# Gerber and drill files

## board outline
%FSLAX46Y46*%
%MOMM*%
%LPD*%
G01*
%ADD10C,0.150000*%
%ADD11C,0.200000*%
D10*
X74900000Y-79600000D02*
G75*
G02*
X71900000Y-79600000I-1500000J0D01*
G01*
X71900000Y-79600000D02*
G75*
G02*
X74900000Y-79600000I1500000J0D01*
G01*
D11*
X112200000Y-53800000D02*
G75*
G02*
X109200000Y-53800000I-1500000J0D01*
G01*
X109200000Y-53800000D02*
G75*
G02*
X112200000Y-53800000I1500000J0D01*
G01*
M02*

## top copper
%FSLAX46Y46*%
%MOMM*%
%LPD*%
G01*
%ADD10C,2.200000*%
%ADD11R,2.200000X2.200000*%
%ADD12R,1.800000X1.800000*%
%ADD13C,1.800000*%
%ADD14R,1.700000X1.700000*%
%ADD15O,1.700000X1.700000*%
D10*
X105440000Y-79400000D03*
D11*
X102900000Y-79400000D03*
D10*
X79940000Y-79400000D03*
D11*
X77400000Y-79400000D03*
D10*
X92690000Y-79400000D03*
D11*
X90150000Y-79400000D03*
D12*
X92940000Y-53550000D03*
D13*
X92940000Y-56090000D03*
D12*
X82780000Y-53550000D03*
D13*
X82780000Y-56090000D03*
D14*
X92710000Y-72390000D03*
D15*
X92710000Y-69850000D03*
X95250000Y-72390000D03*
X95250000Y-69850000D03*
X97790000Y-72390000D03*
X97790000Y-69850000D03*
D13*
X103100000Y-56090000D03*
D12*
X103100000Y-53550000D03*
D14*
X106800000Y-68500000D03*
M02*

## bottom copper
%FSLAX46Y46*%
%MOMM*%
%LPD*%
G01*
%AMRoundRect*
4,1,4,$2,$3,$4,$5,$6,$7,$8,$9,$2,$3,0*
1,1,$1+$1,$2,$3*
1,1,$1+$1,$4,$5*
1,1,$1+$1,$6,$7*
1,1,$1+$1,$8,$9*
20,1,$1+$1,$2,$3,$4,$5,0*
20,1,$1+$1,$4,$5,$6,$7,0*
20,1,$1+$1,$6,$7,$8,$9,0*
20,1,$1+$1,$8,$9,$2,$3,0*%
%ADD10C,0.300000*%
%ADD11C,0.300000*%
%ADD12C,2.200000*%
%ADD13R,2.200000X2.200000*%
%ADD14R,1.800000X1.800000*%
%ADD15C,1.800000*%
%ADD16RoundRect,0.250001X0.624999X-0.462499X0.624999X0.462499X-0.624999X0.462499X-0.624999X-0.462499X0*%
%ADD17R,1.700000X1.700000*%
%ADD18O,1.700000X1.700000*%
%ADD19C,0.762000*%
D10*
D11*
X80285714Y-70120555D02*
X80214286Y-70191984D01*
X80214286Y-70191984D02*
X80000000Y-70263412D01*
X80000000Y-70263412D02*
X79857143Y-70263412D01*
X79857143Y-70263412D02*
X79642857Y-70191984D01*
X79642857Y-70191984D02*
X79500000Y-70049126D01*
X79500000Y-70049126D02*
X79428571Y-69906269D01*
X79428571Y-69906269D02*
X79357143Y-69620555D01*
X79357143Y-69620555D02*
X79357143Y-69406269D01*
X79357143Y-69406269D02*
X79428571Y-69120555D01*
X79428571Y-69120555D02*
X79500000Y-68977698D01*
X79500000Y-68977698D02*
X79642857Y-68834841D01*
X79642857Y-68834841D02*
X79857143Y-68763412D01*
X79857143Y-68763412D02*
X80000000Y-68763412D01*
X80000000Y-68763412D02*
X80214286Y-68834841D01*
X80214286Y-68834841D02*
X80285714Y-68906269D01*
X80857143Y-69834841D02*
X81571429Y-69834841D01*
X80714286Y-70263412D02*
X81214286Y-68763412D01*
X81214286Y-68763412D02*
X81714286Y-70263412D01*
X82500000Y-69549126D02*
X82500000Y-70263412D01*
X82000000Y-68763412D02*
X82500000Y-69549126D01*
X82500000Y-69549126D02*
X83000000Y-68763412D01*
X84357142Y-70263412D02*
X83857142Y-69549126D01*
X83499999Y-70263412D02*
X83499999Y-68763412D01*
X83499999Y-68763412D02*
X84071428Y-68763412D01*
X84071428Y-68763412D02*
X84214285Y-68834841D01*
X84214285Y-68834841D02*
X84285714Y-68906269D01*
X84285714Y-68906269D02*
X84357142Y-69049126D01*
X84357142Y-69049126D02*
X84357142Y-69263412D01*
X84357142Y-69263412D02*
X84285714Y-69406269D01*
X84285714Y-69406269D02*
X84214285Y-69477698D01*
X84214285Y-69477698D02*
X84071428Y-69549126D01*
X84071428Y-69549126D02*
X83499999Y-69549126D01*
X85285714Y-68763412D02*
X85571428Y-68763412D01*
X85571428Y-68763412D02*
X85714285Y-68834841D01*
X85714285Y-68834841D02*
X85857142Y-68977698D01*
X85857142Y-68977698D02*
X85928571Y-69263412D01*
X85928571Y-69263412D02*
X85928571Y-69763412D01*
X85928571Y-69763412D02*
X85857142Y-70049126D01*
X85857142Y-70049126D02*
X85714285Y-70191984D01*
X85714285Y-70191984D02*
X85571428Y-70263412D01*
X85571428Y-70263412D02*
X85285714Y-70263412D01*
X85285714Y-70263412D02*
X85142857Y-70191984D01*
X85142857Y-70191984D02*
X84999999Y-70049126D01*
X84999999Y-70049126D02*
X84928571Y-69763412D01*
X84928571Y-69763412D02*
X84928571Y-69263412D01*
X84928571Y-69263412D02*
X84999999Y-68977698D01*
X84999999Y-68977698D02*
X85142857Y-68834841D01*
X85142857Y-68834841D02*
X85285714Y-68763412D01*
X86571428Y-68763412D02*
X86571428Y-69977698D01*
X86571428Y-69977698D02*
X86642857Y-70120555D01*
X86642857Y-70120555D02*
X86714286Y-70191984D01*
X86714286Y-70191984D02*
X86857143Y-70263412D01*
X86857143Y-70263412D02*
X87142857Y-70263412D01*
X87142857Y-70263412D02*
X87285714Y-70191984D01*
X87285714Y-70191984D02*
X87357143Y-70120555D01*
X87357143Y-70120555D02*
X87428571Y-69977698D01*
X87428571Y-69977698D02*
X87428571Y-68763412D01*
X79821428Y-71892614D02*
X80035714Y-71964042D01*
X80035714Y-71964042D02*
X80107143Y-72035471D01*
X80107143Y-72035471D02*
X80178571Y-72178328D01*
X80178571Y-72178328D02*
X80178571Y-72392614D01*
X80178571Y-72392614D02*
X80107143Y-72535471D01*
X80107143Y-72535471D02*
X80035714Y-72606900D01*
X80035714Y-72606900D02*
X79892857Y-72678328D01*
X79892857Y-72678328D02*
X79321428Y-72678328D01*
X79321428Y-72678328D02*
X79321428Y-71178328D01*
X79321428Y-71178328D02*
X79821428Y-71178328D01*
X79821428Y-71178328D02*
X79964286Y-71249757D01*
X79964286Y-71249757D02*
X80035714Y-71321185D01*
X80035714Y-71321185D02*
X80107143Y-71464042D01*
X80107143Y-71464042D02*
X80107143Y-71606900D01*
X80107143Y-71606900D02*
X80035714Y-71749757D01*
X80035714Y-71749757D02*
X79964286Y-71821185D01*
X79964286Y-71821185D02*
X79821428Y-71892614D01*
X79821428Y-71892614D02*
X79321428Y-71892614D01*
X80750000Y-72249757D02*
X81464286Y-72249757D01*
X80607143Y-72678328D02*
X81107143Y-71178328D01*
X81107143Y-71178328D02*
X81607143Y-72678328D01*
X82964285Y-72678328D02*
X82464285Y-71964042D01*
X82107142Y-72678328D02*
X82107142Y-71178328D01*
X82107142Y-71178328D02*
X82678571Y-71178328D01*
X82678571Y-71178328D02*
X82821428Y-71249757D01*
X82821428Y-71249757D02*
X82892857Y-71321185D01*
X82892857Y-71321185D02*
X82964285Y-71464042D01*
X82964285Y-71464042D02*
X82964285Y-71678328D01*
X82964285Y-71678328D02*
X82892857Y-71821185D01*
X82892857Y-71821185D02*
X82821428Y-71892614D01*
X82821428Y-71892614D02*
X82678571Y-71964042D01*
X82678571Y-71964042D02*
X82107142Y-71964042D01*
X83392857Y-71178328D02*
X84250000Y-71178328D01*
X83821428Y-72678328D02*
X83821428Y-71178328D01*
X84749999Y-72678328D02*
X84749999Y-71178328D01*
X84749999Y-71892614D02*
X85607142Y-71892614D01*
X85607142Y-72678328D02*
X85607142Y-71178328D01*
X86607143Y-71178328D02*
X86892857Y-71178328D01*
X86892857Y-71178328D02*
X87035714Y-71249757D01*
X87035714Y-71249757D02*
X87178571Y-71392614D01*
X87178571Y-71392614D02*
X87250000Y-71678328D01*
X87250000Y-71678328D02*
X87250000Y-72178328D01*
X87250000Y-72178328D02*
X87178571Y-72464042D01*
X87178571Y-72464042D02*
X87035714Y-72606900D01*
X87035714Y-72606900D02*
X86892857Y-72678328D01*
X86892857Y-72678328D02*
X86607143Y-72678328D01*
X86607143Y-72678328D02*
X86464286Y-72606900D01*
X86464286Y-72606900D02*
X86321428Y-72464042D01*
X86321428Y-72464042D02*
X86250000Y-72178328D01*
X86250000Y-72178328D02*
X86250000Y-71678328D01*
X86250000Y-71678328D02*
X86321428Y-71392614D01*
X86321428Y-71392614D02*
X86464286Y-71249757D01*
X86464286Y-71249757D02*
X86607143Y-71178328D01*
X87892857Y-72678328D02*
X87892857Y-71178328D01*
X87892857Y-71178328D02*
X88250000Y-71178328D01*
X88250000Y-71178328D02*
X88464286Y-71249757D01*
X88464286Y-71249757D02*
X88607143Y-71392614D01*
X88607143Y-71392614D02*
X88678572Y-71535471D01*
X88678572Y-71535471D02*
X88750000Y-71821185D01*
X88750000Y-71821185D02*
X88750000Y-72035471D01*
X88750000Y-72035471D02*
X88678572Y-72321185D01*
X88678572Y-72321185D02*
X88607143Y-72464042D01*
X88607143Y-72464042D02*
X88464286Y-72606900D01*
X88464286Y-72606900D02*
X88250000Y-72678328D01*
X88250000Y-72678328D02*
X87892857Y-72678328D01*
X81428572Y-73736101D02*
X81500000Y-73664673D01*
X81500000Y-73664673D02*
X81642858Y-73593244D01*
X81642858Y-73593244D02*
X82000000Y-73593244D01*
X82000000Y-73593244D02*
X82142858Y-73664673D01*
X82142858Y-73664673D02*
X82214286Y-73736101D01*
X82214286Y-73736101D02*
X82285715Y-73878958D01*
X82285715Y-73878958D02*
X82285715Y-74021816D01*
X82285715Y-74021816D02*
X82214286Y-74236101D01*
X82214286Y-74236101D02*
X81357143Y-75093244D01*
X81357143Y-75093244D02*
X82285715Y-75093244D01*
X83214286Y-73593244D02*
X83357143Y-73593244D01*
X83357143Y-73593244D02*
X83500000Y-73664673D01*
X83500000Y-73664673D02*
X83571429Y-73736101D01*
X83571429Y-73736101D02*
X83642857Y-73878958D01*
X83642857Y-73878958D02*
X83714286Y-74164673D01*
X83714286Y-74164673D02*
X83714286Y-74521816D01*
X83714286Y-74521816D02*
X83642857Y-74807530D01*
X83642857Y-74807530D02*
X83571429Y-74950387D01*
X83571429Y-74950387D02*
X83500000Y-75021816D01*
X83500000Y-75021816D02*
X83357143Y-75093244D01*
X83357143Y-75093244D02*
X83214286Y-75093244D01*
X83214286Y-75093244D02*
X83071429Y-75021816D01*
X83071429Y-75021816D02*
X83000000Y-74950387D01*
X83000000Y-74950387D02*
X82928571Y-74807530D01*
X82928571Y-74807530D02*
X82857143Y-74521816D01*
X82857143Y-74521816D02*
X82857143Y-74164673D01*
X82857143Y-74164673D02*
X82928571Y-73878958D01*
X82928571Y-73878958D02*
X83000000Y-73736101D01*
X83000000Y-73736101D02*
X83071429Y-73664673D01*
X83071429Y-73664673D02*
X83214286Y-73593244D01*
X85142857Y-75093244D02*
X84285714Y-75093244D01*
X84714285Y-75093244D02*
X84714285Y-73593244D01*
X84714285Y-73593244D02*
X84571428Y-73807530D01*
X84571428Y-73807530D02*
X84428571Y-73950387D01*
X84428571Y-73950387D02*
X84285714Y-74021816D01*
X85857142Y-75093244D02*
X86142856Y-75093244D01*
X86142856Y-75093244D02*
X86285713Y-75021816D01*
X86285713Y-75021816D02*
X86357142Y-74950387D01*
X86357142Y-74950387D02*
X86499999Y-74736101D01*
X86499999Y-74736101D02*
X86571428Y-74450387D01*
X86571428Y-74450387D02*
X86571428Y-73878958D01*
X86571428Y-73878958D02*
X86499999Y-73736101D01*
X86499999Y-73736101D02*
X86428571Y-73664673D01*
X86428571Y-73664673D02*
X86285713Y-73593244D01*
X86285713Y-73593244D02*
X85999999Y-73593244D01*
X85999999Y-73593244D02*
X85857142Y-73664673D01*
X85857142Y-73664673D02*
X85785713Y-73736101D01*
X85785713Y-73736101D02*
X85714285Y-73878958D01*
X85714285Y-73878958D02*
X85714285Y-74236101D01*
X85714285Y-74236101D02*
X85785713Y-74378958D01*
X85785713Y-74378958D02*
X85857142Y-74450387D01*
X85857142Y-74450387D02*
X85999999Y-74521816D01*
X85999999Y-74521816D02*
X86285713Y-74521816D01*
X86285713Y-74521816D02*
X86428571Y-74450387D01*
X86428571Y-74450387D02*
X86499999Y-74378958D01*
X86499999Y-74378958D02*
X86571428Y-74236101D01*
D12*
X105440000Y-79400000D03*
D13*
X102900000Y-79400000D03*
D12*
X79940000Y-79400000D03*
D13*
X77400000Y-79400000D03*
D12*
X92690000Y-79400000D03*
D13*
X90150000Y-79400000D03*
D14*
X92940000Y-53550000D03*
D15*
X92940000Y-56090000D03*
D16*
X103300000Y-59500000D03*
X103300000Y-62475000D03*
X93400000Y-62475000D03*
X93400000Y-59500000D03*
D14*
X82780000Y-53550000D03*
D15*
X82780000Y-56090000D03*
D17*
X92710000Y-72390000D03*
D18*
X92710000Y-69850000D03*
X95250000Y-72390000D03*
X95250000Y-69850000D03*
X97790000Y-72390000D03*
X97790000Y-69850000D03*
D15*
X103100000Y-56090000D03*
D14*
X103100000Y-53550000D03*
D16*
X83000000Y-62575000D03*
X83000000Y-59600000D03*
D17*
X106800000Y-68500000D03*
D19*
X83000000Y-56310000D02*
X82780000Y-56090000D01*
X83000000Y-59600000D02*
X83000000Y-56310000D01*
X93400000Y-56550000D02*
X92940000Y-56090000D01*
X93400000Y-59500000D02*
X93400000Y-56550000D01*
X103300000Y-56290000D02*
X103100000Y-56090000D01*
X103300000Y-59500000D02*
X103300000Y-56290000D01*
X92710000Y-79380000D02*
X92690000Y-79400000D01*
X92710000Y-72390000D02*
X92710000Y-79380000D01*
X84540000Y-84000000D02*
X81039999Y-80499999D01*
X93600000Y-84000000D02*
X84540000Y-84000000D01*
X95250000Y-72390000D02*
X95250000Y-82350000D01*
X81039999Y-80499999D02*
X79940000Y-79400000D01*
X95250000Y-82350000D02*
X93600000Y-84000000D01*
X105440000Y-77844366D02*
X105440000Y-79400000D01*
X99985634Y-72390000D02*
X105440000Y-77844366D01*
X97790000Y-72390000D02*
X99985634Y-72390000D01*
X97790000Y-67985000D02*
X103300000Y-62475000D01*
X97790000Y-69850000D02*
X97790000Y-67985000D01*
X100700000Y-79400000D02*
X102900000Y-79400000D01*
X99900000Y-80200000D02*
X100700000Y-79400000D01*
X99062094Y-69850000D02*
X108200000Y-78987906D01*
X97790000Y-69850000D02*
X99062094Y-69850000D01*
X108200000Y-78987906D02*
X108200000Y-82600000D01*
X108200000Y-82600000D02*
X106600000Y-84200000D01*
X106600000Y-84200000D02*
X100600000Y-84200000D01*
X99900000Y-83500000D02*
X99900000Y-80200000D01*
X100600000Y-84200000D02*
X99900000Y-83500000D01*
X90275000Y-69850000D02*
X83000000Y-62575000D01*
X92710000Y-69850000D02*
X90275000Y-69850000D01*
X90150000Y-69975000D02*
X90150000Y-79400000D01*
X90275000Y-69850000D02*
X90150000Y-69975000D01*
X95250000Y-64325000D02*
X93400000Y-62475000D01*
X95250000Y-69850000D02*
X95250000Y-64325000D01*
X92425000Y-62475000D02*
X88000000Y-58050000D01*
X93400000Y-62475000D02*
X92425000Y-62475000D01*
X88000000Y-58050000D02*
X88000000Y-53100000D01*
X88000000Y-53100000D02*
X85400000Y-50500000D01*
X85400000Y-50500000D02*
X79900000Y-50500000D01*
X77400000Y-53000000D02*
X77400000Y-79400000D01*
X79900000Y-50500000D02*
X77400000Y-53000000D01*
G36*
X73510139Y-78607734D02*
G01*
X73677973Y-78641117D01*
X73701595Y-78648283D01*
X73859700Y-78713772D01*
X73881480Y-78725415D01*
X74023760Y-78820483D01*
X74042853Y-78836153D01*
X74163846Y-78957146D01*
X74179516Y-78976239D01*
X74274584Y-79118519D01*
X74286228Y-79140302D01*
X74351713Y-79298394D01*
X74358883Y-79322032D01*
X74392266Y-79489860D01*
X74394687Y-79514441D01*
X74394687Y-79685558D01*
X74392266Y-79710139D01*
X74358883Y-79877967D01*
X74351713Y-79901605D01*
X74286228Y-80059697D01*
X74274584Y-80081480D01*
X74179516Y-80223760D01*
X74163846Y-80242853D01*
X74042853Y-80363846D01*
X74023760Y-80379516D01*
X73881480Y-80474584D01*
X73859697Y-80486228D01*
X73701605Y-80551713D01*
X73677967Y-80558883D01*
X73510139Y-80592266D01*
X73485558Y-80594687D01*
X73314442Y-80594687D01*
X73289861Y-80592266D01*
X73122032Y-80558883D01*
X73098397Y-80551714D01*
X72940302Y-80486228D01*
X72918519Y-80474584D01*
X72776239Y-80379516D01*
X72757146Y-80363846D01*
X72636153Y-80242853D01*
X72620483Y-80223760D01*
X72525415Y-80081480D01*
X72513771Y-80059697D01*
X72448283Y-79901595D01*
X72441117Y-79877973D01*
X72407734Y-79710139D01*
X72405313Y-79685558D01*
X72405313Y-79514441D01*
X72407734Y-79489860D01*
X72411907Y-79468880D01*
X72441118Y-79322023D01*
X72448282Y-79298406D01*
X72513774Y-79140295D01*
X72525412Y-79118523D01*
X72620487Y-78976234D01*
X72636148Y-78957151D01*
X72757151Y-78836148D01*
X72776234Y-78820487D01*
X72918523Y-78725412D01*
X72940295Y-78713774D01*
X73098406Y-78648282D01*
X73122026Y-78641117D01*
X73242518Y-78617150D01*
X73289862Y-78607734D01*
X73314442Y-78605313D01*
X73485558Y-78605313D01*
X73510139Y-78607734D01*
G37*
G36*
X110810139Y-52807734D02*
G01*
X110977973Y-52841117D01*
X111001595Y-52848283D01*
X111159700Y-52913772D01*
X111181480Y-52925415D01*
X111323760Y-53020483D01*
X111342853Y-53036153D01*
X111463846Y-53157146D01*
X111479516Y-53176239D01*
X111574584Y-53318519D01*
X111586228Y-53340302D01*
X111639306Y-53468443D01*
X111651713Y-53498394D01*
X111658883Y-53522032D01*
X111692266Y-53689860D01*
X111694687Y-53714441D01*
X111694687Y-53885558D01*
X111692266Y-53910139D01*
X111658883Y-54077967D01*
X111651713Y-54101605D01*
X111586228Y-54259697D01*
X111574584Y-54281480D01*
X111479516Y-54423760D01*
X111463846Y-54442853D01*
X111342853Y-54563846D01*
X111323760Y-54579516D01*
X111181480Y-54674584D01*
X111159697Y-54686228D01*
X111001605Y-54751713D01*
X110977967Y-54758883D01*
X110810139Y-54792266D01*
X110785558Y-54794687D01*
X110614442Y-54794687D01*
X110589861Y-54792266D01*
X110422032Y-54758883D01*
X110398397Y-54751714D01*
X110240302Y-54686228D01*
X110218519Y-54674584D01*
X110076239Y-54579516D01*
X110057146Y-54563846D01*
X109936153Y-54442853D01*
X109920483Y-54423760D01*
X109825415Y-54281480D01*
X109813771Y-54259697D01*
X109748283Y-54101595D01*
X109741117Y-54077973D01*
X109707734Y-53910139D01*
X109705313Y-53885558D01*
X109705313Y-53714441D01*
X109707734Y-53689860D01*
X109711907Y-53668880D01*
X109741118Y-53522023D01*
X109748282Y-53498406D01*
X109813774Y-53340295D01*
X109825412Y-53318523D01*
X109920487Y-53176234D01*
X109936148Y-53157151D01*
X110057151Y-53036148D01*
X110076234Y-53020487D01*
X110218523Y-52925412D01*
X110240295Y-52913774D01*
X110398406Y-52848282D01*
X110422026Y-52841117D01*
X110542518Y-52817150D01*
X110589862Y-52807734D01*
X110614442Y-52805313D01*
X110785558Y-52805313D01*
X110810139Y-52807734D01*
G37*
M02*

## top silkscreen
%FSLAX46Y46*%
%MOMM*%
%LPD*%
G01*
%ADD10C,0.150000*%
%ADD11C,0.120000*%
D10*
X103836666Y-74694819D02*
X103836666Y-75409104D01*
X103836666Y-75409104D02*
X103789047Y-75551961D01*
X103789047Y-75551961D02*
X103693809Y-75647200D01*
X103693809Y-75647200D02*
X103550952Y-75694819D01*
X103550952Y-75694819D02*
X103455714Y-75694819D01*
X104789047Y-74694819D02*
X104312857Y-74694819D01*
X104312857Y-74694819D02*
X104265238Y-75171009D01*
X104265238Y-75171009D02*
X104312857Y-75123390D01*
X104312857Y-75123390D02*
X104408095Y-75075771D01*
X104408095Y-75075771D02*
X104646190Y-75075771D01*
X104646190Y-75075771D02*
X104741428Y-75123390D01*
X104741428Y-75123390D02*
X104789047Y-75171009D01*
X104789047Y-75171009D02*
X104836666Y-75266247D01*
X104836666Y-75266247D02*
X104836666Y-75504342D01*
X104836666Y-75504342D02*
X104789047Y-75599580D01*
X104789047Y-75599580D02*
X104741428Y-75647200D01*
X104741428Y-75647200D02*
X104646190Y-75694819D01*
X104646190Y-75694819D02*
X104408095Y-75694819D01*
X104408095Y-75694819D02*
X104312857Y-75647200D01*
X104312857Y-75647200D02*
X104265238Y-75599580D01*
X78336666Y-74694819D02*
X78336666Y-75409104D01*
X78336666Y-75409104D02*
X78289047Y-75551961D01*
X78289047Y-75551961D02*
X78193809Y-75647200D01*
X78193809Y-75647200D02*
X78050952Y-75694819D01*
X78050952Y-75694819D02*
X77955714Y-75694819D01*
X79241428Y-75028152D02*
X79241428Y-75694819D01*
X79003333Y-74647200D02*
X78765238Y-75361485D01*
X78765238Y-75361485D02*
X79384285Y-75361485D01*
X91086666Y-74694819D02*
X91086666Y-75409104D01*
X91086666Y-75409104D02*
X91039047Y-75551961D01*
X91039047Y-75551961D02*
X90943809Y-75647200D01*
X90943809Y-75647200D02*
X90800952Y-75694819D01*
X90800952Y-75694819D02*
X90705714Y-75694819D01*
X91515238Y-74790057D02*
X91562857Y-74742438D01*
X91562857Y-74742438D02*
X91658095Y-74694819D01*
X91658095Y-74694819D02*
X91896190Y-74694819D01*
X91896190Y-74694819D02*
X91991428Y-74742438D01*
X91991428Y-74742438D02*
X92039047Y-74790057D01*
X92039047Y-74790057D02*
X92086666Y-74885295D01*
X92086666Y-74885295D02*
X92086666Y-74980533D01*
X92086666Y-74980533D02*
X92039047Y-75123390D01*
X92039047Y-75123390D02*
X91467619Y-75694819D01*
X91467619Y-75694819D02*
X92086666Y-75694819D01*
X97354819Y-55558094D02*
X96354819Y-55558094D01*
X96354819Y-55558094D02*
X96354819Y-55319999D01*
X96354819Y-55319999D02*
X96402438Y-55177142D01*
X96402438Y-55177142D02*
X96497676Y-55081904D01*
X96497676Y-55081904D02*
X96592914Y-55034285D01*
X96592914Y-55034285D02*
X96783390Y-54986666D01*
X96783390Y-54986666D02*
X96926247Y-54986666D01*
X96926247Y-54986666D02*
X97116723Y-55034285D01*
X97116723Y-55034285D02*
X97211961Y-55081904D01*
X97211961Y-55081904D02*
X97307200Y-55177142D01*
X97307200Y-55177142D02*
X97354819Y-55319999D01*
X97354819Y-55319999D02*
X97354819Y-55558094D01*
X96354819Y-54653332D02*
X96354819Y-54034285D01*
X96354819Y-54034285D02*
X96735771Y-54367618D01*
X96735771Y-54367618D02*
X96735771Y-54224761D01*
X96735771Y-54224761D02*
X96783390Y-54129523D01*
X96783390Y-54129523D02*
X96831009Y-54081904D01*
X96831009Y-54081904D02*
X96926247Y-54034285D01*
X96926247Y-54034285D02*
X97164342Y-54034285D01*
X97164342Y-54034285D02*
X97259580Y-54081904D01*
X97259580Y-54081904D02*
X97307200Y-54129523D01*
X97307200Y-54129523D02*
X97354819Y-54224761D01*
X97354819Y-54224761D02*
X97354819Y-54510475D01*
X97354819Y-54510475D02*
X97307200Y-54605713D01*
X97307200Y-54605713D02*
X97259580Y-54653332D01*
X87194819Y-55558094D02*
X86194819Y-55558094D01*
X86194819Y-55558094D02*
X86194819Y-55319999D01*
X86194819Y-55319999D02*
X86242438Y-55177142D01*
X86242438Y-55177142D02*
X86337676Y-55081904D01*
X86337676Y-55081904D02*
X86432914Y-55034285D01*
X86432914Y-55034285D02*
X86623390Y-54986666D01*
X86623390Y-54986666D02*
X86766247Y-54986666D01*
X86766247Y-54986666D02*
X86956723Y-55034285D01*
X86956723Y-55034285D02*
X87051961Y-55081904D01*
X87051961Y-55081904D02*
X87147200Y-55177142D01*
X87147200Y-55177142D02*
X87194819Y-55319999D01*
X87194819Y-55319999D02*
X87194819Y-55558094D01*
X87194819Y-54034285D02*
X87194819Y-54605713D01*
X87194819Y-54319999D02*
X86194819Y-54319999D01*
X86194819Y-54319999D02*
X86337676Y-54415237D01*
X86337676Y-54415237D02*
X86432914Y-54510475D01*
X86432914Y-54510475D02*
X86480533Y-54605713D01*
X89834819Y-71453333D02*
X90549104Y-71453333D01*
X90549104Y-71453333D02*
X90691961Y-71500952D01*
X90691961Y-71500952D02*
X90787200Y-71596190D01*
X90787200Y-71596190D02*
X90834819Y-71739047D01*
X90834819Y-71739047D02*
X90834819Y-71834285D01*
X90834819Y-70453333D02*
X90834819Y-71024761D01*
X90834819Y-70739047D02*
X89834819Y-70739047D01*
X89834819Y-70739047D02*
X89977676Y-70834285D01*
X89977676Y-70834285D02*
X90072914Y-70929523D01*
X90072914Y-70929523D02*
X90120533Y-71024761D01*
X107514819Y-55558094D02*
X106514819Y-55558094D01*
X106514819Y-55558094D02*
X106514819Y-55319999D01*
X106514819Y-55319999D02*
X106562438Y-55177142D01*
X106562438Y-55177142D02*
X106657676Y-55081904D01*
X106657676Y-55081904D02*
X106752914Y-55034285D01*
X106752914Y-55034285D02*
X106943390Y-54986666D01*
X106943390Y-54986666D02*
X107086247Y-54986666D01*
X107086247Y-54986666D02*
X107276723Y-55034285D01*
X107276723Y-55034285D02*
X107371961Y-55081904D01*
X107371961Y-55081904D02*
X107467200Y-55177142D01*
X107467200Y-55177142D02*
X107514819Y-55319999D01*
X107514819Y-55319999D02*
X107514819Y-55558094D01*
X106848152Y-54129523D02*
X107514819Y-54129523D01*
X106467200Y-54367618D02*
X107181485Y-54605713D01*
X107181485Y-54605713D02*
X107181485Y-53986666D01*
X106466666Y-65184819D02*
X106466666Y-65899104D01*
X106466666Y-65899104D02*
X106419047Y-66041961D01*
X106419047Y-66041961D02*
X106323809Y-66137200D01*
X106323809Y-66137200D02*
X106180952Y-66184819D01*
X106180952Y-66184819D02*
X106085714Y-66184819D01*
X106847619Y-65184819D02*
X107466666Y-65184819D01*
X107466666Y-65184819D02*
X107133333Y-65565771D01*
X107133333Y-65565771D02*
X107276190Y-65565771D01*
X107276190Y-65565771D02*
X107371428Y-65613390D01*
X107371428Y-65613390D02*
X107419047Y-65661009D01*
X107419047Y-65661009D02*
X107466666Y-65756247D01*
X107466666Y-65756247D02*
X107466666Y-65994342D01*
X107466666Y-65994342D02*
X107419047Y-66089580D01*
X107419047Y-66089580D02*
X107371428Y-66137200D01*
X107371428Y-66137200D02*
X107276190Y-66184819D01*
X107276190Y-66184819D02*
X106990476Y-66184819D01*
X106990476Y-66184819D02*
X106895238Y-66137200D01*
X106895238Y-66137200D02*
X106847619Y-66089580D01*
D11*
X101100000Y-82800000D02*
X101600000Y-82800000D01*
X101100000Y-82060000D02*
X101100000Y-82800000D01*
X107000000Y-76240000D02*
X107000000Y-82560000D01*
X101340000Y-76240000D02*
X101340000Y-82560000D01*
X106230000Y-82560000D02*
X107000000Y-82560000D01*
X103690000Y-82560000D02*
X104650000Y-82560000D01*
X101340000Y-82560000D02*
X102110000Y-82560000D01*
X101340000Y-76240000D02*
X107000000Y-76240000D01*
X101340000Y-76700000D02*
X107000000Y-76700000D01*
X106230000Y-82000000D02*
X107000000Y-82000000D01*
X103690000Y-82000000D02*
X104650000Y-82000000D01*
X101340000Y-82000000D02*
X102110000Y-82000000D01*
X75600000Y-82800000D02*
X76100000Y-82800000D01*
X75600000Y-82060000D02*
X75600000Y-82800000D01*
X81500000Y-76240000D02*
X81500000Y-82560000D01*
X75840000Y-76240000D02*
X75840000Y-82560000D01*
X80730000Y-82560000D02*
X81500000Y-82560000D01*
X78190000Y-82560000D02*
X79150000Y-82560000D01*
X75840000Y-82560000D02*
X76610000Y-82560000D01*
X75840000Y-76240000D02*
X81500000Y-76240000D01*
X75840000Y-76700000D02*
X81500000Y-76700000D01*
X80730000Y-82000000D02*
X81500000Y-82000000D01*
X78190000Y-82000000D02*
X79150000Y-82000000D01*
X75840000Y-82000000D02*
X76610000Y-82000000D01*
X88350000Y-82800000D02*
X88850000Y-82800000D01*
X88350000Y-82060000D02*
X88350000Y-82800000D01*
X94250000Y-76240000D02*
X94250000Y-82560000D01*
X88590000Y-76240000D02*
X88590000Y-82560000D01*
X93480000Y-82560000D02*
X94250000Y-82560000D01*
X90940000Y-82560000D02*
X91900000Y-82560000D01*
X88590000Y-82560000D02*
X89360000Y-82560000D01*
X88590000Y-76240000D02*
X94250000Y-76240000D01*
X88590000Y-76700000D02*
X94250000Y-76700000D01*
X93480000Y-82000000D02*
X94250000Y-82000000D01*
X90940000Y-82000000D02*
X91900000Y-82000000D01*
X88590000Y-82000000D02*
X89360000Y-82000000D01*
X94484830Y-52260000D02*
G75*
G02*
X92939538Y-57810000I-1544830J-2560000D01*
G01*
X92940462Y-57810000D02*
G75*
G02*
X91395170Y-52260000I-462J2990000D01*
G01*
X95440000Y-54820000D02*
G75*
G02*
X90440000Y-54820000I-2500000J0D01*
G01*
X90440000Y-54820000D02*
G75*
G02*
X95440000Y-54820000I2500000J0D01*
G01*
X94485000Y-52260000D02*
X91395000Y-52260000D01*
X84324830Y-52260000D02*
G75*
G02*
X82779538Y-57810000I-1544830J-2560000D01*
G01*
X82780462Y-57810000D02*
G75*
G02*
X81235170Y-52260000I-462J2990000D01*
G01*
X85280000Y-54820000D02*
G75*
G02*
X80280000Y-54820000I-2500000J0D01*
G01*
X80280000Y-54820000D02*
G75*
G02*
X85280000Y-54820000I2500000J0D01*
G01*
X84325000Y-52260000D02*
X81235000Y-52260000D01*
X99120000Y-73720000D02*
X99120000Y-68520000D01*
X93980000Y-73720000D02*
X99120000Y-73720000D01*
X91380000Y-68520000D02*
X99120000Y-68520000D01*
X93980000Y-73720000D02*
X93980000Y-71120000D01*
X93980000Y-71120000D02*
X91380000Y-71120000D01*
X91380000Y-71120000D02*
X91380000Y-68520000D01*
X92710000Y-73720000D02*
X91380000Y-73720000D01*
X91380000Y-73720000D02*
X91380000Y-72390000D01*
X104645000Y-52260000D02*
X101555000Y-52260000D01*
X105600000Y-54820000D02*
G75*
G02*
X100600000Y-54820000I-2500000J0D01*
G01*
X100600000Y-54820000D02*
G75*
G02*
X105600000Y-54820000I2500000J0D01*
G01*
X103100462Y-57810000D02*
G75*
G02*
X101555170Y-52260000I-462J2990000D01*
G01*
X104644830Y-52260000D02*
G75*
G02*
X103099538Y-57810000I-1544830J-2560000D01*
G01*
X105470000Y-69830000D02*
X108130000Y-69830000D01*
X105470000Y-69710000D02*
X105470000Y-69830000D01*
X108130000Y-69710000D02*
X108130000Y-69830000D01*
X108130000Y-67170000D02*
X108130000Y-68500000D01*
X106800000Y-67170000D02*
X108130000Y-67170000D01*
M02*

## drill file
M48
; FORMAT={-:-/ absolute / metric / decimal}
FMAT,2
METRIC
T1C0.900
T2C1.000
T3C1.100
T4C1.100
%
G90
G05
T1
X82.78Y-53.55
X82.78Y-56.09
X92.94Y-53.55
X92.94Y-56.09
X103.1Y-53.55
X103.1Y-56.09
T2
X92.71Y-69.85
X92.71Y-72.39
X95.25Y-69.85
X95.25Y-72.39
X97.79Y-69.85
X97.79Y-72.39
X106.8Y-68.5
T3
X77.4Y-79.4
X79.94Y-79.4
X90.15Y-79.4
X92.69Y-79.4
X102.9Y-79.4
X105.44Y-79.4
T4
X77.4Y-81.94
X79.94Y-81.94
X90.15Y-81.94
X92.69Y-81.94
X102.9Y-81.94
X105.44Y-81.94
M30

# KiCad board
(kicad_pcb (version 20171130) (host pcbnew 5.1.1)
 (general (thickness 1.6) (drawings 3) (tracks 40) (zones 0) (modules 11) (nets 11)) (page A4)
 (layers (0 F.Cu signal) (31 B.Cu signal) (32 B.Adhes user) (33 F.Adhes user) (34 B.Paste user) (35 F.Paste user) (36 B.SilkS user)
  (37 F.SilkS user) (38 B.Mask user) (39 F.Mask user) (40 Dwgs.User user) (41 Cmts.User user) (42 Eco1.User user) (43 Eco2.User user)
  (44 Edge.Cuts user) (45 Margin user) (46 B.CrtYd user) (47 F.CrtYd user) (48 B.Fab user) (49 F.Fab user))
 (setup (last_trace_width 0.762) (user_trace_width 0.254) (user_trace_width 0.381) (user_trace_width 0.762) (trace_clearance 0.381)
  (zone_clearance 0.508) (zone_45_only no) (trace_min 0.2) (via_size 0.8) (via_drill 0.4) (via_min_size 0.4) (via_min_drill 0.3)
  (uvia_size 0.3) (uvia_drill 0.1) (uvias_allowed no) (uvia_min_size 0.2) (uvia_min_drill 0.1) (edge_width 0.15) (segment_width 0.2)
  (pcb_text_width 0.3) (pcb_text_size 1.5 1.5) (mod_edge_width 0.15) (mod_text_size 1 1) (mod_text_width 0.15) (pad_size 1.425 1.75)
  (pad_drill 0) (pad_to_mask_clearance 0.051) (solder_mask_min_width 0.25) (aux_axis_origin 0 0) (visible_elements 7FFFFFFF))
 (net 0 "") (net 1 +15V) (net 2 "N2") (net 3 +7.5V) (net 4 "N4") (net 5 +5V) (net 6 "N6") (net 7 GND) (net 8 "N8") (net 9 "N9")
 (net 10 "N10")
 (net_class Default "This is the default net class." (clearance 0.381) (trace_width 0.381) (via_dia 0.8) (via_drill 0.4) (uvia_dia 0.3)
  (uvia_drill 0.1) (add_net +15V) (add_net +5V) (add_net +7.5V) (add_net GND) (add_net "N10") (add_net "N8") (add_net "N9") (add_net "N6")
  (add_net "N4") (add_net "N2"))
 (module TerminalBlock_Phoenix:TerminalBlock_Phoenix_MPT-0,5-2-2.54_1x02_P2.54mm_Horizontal (layer F.Cu) (at 102.9 79.4)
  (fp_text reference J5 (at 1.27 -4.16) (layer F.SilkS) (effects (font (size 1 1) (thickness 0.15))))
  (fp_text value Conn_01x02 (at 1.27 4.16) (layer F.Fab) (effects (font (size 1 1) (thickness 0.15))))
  (fp_line (start -1.8 3.4) (end -1.3 3.4) (layer F.SilkS) (width 0.12))
  (fp_line (start -1.8 2.66) (end -1.8 3.4) (layer F.SilkS) (width 0.12))
  (fp_line (start 4.1 -3.16) (end 4.1 3.16) (layer F.SilkS) (width 0.12))
  (fp_line (start -1.56 -3.16) (end -1.56 3.16) (layer F.SilkS) (width 0.12))
  (fp_line (start 3.33 3.16) (end 4.1 3.16) (layer F.SilkS) (width 0.12))
  (fp_line (start 0.79 3.16) (end 1.75 3.16) (layer F.SilkS) (width 0.12))
  (fp_line (start -1.56 3.16) (end -0.79 3.16) (layer F.SilkS) (width 0.12))
  (fp_line (start -1.56 -3.16) (end 4.1 -3.16) (layer F.SilkS) (width 0.12))
  (fp_line (start -1.56 -2.7) (end 4.1 -2.7) (layer F.SilkS) (width 0.12))
  (fp_line (start 3.33 2.6) (end 4.1 2.6) (layer F.SilkS) (width 0.12))
  (fp_line (start 0.79 2.6) (end 1.75 2.6) (layer F.SilkS) (width 0.12))
  (fp_line (start -1.56 2.6) (end -0.79 2.6) (layer F.SilkS) (width 0.12))
  (pad "" np_thru_hole circle (at 2.54 2.54) (size 1.1 1.1) (drill 1.1) (layers *.Cu *.Mask))
  (pad 2 thru_hole circle (at 2.54 0) (size 2.2 2.2) (drill 1.1) (layers *.Cu *.Mask) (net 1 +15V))
  (pad "" np_thru_hole circle (at 0 2.54) (size 1.1 1.1) (drill 1.1) (layers *.Cu *.Mask))
  (pad 1 thru_hole rect (at 0 0) (size 2.2 2.2) (drill 1.1) (layers *.Cu *.Mask) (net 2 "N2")))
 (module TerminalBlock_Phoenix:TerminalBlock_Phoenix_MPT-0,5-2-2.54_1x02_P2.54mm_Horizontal (layer F.Cu) (at 77.4 79.4)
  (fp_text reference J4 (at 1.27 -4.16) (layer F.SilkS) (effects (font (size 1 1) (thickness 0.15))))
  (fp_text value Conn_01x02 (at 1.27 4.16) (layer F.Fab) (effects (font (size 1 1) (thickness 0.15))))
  (fp_line (start -1.8 3.4) (end -1.3 3.4) (layer F.SilkS) (width 0.12))
  (fp_line (start -1.8 2.66) (end -1.8 3.4) (layer F.SilkS) (width 0.12))
  (fp_line (start 4.1 -3.16) (end 4.1 3.16) (layer F.SilkS) (width 0.12))
  (fp_line (start -1.56 -3.16) (end -1.56 3.16) (layer F.SilkS) (width 0.12))
  (fp_line (start 3.33 3.16) (end 4.1 3.16) (layer F.SilkS) (width 0.12))
  (fp_line (start 0.79 3.16) (end 1.75 3.16) (layer F.SilkS) (width 0.12))
  (fp_line (start -1.56 3.16) (end -0.79 3.16) (layer F.SilkS) (width 0.12))
  (fp_line (start -1.56 -3.16) (end 4.1 -3.16) (layer F.SilkS) (width 0.12))
  (fp_line (start -1.56 -2.7) (end 4.1 -2.7) (layer F.SilkS) (width 0.12))
  (fp_line (start 3.33 2.6) (end 4.1 2.6) (layer F.SilkS) (width 0.12))
  (fp_line (start 0.79 2.6) (end 1.75 2.6) (layer F.SilkS) (width 0.12))
  (fp_line (start -1.56 2.6) (end -0.79 2.6) (layer F.SilkS) (width 0.12))
  (pad "" np_thru_hole circle (at 2.54 2.54) (size 1.1 1.1) (drill 1.1) (layers *.Cu *.Mask))
  (pad 2 thru_hole circle (at 2.54 0) (size 2.2 2.2) (drill 1.1) (layers *.Cu *.Mask) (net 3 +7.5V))
  (pad "" np_thru_hole circle (at 0 2.54) (size 1.1 1.1) (drill 1.1) (layers *.Cu *.Mask))
  (pad 1 thru_hole rect (at 0 0) (size 2.2 2.2) (drill 1.1) (layers *.Cu *.Mask) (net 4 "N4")))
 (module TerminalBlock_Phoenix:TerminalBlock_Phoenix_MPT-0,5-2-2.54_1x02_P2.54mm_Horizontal (layer F.Cu) (at 90.15 79.4)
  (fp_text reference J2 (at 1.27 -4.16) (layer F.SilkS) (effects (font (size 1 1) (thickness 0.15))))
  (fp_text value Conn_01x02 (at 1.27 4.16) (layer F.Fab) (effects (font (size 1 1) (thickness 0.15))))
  (fp_line (start -1.8 3.4) (end -1.3 3.4) (layer F.SilkS) (width 0.12))
  (fp_line (start -1.8 2.66) (end -1.8 3.4) (layer F.SilkS) (width 0.12))
  (fp_line (start 4.1 -3.16) (end 4.1 3.16) (layer F.SilkS) (width 0.12))
  (fp_line (start -1.56 -3.16) (end -1.56 3.16) (layer F.SilkS) (width 0.12))
  (fp_line (start 3.33 3.16) (end 4.1 3.16) (layer F.SilkS) (width 0.12))
  (fp_line (start 0.79 3.16) (end 1.75 3.16) (layer F.SilkS) (width 0.12))
  (fp_line (start -1.56 3.16) (end -0.79 3.16) (layer F.SilkS) (width 0.12))
  (fp_line (start -1.56 -3.16) (end 4.1 -3.16) (layer F.SilkS) (width 0.12))
  (fp_line (start -1.56 -2.7) (end 4.1 -2.7) (layer F.SilkS) (width 0.12))
  (fp_line (start 3.33 2.6) (end 4.1 2.6) (layer F.SilkS) (width 0.12))
  (fp_line (start 0.79 2.6) (end 1.75 2.6) (layer F.SilkS) (width 0.12))
  (fp_line (start -1.56 2.6) (end -0.79 2.6) (layer F.SilkS) (width 0.12))
  (pad "" np_thru_hole circle (at 2.54 2.54) (size 1.1 1.1) (drill 1.1) (layers *.Cu *.Mask))
  (pad 2 thru_hole circle (at 2.54 0) (size 2.2 2.2) (drill 1.1) (layers *.Cu *.Mask) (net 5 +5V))
  (pad "" np_thru_hole circle (at 0 2.54) (size 1.1 1.1) (drill 1.1) (layers *.Cu *.Mask))
  (pad 1 thru_hole rect (at 0 0) (size 2.2 2.2) (drill 1.1) (layers *.Cu *.Mask) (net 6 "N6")))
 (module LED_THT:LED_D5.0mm (layer F.Cu) (at 92.94 53.55 270)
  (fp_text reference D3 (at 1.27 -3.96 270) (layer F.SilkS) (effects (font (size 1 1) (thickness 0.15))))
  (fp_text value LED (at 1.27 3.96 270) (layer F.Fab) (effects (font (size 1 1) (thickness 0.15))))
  (fp_arc (start 1.27 0) (end -1.29 -1.54483) (angle 148.9) (layer F.SilkS) (width 0.12))
  (fp_arc (start 1.27 0) (end -1.29 1.54483) (angle -148.9) (layer F.SilkS) (width 0.12))
  (fp_circle (center 1.27 0) (end 3.77 0) (layer F.SilkS) (width 0.12))
  (fp_line (start -1.29 -1.545) (end -1.29 1.545) (layer F.SilkS) (width 0.12))
  (pad 1 thru_hole rect (at 0 0 270) (size 1.8 1.8) (drill 0.9) (layers *.Cu *.Mask) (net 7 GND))
  (pad 2 thru_hole circle (at 2.54 0 270) (size 1.8 1.8) (drill 0.9) (layers *.Cu *.Mask) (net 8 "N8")))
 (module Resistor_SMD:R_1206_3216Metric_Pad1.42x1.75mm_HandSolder (layer B.Cu) (at 103.3 60.9875 90)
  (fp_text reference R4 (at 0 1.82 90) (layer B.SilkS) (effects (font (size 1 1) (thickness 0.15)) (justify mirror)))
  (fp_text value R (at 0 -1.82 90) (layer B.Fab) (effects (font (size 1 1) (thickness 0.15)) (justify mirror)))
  (pad 2 smd roundrect (at 1.4875 0 90) (size 1.425 1.75) (layers B.Cu B.Paste B.Mask) (roundrect_rratio 0.175439) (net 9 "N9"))
  (pad 1 smd roundrect (at -1.4875 0 90) (size 1.425 1.75) (layers B.Cu B.Paste B.Mask) (roundrect_rratio 0.175439) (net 2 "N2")))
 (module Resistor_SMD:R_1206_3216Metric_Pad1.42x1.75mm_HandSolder (layer B.Cu) (at 93.4 60.9875 90)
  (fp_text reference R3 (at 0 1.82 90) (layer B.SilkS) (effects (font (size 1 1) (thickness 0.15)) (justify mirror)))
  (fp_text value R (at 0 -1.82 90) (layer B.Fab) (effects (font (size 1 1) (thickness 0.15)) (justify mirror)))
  (pad 1 smd roundrect (at -1.4875 0 90) (size 1.425 1.75) (layers B.Cu B.Paste B.Mask) (roundrect_rratio 0.175439) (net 4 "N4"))
  (pad 2 smd roundrect (at 1.4875 0 90) (size 1.425 1.75) (layers B.Cu B.Paste B.Mask) (roundrect_rratio 0.175439) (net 8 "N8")))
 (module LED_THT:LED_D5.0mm (layer F.Cu) (at 82.78 53.55 270)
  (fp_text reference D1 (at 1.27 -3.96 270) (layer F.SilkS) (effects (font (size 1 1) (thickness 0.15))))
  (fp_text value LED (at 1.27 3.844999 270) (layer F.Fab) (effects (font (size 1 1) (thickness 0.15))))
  (fp_arc (start 1.27 0) (end -1.29 -1.54483) (angle 148.9) (layer F.SilkS) (width 0.12))
  (fp_arc (start 1.27 0) (end -1.29 1.54483) (angle -148.9) (layer F.SilkS) (width 0.12))
  (fp_circle (center 1.27 0) (end 3.77 0) (layer F.SilkS) (width 0.12))
  (fp_line (start -1.29 -1.545) (end -1.29 1.545) (layer F.SilkS) (width 0.12))
  (pad 1 thru_hole rect (at 0 0 270) (size 1.8 1.8) (drill 0.9) (layers *.Cu *.Mask) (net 7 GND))
  (pad 2 thru_hole circle (at 2.54 0 270) (size 1.8 1.8) (drill 0.9) (layers *.Cu *.Mask) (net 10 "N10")))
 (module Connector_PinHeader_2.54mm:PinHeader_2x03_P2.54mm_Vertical (layer F.Cu) (at 92.71 72.39 90)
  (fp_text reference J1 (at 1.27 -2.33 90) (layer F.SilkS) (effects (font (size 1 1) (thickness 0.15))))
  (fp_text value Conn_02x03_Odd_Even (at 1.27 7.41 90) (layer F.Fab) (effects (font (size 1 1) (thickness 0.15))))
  (fp_line (start -1.33 6.41) (end 3.87 6.41) (layer F.SilkS) (width 0.12))
  (fp_line (start -1.33 1.27) (end -1.33 6.41) (layer F.SilkS) (width 0.12))
  (fp_line (start 3.87 -1.33) (end 3.87 6.41) (layer F.SilkS) (width 0.12))
  (fp_line (start -1.33 1.27) (end 1.27 1.27) (layer F.SilkS) (width 0.12))
  (fp_line (start 1.27 1.27) (end 1.27 -1.33) (layer F.SilkS) (width 0.12))
  (fp_line (start 1.27 -1.33) (end 3.87 -1.33) (layer F.SilkS) (width 0.12))
  (fp_line (start -1.33 0) (end -1.33 -1.33) (layer F.SilkS) (width 0.12))
  (fp_line (start -1.33 -1.33) (end 0 -1.33) (layer F.SilkS) (width 0.12))
  (pad 1 thru_hole rect (at 0 0 90) (size 1.7 1.7) (drill 1) (layers *.Cu *.Mask) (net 5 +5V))
  (pad 2 thru_hole oval (at 2.54 0 90) (size 1.7 1.7) (drill 1) (layers *.Cu *.Mask) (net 6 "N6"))
  (pad 3 thru_hole oval (at 0 2.54 90) (size 1.7 1.7) (drill 1) (layers *.Cu *.Mask) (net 3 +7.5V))
  (pad 4 thru_hole oval (at 2.54 2.54 90) (size 1.7 1.7) (drill 1) (layers *.Cu *.Mask) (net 4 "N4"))
  (pad 5 thru_hole oval (at 0 5.08 90) (size 1.7 1.7) (drill 1) (layers *.Cu *.Mask) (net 1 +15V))
  (pad 6 thru_hole oval (at 2.54 5.08 90) (size 1.7 1.7) (drill 1) (layers *.Cu *.Mask) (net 2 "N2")))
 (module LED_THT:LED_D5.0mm (layer F.Cu) (at 103.1 53.55 270)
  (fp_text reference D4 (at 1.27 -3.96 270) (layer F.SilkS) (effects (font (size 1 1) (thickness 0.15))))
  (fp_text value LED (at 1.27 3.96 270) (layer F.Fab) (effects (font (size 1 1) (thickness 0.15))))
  (fp_line (start -1.29 -1.545) (end -1.29 1.545) (layer F.SilkS) (width 0.12))
  (fp_circle (center 1.27 0) (end 3.77 0) (layer F.SilkS) (width 0.12))
  (fp_arc (start 1.27 0) (end -1.29 1.54483) (angle -148.9) (layer F.SilkS) (width 0.12))
  (fp_arc (start 1.27 0) (end -1.29 -1.54483) (angle 148.9) (layer F.SilkS) (width 0.12))
  (pad 2 thru_hole circle (at 2.54 0 270) (size 1.8 1.8) (drill 0.9) (layers *.Cu *.Mask) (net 9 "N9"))
  (pad 1 thru_hole rect (at 0 0 270) (size 1.8 1.8) (drill 0.9) (layers *.Cu *.Mask) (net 7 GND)))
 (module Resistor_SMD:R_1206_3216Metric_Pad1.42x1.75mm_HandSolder (layer B.Cu) (at 83 61.0875 90)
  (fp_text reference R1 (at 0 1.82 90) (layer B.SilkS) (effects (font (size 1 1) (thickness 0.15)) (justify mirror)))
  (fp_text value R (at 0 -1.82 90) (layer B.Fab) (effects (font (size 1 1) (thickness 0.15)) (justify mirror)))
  (pad 1 smd roundrect (at -1.4875 0 90) (size 1.425 1.75) (layers B.Cu B.Paste B.Mask) (roundrect_rratio 0.175439) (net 6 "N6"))
  (pad 2 smd roundrect (at 1.4875 0 90) (size 1.425 1.75) (layers B.Cu B.Paste B.Mask) (roundrect_rratio 0.175439) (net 10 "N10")))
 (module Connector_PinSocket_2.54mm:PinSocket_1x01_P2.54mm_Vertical (layer F.Cu) (at 106.8 68.5)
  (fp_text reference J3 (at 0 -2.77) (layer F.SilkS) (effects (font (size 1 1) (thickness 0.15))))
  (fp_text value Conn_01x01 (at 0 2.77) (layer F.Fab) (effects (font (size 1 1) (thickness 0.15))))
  (fp_line (start -1.33 1.33) (end 1.33 1.33) (layer F.SilkS) (width 0.12))
  (fp_line (start -1.33 1.21) (end -1.33 1.33) (layer F.SilkS) (width 0.12))
  (fp_line (start 1.33 1.21) (end 1.33 1.33) (layer F.SilkS) (width 0.12))
  (fp_line (start 1.33 -1.33) (end 1.33 0) (layer F.SilkS) (width 0.12))
  (fp_line (start 0 -1.33) (end 1.33 -1.33) (layer F.SilkS) (width 0.12))
  (pad 1 thru_hole rect (at 0 0) (size 1.7 1.7) (drill 1) (layers *.Cu *.Mask) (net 7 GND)))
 (gr_circle (center 73.4 79.6) (end 74.9 79.6) (layer Edge.Cuts) (width 0.15))
 (gr_circle (center 110.7 53.8) (end 112.2 53.8) (layer Edge.Cuts) (width 0.2))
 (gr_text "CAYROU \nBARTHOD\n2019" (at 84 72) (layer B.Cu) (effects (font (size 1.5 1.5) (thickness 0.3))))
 (segment (start 83 56.31) (end 82.78 56.09) (width 0.762) (layer B.Cu) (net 10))
 (segment (start 83 59.6) (end 83 56.31) (width 0.762) (layer B.Cu) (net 10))
 (segment (start 93.4 56.55) (end 92.94 56.09) (width 0.762) (layer B.Cu) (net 8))
 (segment (start 93.4 59.5) (end 93.4 56.55) (width 0.762) (layer B.Cu) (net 8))
 (segment (start 103.3 56.29) (end 103.1 56.09) (width 0.762) (layer B.Cu) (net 9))
 (segment (start 103.3 59.5) (end 103.3 56.29) (width 0.762) (layer B.Cu) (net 9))
 (segment (start 92.71 79.38) (end 92.69 79.4) (width 0.762) (layer B.Cu) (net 5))
 (segment (start 92.71 72.39) (end 92.71 79.38) (width 0.762) (layer B.Cu) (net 5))
 (segment (start 84.54 84) (end 81.039999 80.499999) (width 0.762) (layer B.Cu) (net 3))
 (segment (start 93.6 84) (end 84.54 84) (width 0.762) (layer B.Cu) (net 3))
 (segment (start 95.25 72.39) (end 95.25 82.35) (width 0.762) (layer B.Cu) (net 3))
 (segment (start 81.039999 80.499999) (end 79.94 79.4) (width 0.762) (layer B.Cu) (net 3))
 (segment (start 95.25 82.35) (end 93.6 84) (width 0.762) (layer B.Cu) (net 3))
 (segment (start 105.44 77.844366) (end 105.44 79.4) (width 0.762) (layer B.Cu) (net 1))
 (segment (start 99.985634 72.39) (end 105.44 77.844366) (width 0.762) (layer B.Cu) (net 1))
 (segment (start 97.79 72.39) (end 99.985634 72.39) (width 0.762) (layer B.Cu) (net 1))
 (segment (start 97.79 67.985) (end 103.3 62.475) (width 0.762) (layer B.Cu) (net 2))
 (segment (start 97.79 69.85) (end 97.79 67.985) (width 0.762) (layer B.Cu) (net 2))
 (segment (start 100.7 79.4) (end 102.9 79.4) (width 0.762) (layer B.Cu) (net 2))
 (segment (start 99.9 80.2) (end 100.7 79.4) (width 0.762) (layer B.Cu) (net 2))
 (segment (start 99.062094 69.85) (end 108.2 78.987906) (width 0.762) (layer B.Cu) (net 2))
 (segment (start 97.79 69.85) (end 99.062094 69.85) (width 0.762) (layer B.Cu) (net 2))
 (segment (start 108.2 78.987906) (end 108.2 82.6) (width 0.762) (layer B.Cu) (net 2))
 (segment (start 108.2 82.6) (end 106.6 84.2) (width 0.762) (layer B.Cu) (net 2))
 (segment (start 106.6 84.2) (end 100.6 84.2) (width 0.762) (layer B.Cu) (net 2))
 (segment (start 99.9 83.5) (end 99.9 80.2) (width 0.762) (layer B.Cu) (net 2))
 (segment (start 100.6 84.2) (end 99.9 83.5) (width 0.762) (layer B.Cu) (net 2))
 (segment (start 90.275 69.85) (end 83 62.575) (width 0.762) (layer B.Cu) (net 6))
 (segment (start 92.71 69.85) (end 90.275 69.85) (width 0.762) (layer B.Cu) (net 6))
 (segment (start 90.15 69.975) (end 90.15 79.4) (width 0.762) (layer B.Cu) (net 6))
 (segment (start 90.275 69.85) (end 90.15 69.975) (width 0.762) (layer B.Cu) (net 6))
 (segment (start 95.25 64.325) (end 93.4 62.475) (width 0.762) (layer B.Cu) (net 4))
 (segment (start 95.25 69.85) (end 95.25 64.325) (width 0.762) (layer B.Cu) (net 4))
 (segment (start 92.425 62.475) (end 88 58.05) (width 0.762) (layer B.Cu) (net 4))
 (segment (start 93.4 62.475) (end 92.425 62.475) (width 0.762) (layer B.Cu) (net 4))
 (segment (start 88 58.05) (end 88 53.1) (width 0.762) (layer B.Cu) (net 4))
 (segment (start 88 53.1) (end 85.4 50.5) (width 0.762) (layer B.Cu) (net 4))
 (segment (start 85.4 50.5) (end 79.9 50.5) (width 0.762) (layer B.Cu) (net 4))
 (segment (start 77.4 53) (end 77.4 79.4) (width 0.762) (layer B.Cu) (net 4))
 (segment (start 79.9 50.5) (end 77.4 53) (width 0.762) (layer B.Cu) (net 4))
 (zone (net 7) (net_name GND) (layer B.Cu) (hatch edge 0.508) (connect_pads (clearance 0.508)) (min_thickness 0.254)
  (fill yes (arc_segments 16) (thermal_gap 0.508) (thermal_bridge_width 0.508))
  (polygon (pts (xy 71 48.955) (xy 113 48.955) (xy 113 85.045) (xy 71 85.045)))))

